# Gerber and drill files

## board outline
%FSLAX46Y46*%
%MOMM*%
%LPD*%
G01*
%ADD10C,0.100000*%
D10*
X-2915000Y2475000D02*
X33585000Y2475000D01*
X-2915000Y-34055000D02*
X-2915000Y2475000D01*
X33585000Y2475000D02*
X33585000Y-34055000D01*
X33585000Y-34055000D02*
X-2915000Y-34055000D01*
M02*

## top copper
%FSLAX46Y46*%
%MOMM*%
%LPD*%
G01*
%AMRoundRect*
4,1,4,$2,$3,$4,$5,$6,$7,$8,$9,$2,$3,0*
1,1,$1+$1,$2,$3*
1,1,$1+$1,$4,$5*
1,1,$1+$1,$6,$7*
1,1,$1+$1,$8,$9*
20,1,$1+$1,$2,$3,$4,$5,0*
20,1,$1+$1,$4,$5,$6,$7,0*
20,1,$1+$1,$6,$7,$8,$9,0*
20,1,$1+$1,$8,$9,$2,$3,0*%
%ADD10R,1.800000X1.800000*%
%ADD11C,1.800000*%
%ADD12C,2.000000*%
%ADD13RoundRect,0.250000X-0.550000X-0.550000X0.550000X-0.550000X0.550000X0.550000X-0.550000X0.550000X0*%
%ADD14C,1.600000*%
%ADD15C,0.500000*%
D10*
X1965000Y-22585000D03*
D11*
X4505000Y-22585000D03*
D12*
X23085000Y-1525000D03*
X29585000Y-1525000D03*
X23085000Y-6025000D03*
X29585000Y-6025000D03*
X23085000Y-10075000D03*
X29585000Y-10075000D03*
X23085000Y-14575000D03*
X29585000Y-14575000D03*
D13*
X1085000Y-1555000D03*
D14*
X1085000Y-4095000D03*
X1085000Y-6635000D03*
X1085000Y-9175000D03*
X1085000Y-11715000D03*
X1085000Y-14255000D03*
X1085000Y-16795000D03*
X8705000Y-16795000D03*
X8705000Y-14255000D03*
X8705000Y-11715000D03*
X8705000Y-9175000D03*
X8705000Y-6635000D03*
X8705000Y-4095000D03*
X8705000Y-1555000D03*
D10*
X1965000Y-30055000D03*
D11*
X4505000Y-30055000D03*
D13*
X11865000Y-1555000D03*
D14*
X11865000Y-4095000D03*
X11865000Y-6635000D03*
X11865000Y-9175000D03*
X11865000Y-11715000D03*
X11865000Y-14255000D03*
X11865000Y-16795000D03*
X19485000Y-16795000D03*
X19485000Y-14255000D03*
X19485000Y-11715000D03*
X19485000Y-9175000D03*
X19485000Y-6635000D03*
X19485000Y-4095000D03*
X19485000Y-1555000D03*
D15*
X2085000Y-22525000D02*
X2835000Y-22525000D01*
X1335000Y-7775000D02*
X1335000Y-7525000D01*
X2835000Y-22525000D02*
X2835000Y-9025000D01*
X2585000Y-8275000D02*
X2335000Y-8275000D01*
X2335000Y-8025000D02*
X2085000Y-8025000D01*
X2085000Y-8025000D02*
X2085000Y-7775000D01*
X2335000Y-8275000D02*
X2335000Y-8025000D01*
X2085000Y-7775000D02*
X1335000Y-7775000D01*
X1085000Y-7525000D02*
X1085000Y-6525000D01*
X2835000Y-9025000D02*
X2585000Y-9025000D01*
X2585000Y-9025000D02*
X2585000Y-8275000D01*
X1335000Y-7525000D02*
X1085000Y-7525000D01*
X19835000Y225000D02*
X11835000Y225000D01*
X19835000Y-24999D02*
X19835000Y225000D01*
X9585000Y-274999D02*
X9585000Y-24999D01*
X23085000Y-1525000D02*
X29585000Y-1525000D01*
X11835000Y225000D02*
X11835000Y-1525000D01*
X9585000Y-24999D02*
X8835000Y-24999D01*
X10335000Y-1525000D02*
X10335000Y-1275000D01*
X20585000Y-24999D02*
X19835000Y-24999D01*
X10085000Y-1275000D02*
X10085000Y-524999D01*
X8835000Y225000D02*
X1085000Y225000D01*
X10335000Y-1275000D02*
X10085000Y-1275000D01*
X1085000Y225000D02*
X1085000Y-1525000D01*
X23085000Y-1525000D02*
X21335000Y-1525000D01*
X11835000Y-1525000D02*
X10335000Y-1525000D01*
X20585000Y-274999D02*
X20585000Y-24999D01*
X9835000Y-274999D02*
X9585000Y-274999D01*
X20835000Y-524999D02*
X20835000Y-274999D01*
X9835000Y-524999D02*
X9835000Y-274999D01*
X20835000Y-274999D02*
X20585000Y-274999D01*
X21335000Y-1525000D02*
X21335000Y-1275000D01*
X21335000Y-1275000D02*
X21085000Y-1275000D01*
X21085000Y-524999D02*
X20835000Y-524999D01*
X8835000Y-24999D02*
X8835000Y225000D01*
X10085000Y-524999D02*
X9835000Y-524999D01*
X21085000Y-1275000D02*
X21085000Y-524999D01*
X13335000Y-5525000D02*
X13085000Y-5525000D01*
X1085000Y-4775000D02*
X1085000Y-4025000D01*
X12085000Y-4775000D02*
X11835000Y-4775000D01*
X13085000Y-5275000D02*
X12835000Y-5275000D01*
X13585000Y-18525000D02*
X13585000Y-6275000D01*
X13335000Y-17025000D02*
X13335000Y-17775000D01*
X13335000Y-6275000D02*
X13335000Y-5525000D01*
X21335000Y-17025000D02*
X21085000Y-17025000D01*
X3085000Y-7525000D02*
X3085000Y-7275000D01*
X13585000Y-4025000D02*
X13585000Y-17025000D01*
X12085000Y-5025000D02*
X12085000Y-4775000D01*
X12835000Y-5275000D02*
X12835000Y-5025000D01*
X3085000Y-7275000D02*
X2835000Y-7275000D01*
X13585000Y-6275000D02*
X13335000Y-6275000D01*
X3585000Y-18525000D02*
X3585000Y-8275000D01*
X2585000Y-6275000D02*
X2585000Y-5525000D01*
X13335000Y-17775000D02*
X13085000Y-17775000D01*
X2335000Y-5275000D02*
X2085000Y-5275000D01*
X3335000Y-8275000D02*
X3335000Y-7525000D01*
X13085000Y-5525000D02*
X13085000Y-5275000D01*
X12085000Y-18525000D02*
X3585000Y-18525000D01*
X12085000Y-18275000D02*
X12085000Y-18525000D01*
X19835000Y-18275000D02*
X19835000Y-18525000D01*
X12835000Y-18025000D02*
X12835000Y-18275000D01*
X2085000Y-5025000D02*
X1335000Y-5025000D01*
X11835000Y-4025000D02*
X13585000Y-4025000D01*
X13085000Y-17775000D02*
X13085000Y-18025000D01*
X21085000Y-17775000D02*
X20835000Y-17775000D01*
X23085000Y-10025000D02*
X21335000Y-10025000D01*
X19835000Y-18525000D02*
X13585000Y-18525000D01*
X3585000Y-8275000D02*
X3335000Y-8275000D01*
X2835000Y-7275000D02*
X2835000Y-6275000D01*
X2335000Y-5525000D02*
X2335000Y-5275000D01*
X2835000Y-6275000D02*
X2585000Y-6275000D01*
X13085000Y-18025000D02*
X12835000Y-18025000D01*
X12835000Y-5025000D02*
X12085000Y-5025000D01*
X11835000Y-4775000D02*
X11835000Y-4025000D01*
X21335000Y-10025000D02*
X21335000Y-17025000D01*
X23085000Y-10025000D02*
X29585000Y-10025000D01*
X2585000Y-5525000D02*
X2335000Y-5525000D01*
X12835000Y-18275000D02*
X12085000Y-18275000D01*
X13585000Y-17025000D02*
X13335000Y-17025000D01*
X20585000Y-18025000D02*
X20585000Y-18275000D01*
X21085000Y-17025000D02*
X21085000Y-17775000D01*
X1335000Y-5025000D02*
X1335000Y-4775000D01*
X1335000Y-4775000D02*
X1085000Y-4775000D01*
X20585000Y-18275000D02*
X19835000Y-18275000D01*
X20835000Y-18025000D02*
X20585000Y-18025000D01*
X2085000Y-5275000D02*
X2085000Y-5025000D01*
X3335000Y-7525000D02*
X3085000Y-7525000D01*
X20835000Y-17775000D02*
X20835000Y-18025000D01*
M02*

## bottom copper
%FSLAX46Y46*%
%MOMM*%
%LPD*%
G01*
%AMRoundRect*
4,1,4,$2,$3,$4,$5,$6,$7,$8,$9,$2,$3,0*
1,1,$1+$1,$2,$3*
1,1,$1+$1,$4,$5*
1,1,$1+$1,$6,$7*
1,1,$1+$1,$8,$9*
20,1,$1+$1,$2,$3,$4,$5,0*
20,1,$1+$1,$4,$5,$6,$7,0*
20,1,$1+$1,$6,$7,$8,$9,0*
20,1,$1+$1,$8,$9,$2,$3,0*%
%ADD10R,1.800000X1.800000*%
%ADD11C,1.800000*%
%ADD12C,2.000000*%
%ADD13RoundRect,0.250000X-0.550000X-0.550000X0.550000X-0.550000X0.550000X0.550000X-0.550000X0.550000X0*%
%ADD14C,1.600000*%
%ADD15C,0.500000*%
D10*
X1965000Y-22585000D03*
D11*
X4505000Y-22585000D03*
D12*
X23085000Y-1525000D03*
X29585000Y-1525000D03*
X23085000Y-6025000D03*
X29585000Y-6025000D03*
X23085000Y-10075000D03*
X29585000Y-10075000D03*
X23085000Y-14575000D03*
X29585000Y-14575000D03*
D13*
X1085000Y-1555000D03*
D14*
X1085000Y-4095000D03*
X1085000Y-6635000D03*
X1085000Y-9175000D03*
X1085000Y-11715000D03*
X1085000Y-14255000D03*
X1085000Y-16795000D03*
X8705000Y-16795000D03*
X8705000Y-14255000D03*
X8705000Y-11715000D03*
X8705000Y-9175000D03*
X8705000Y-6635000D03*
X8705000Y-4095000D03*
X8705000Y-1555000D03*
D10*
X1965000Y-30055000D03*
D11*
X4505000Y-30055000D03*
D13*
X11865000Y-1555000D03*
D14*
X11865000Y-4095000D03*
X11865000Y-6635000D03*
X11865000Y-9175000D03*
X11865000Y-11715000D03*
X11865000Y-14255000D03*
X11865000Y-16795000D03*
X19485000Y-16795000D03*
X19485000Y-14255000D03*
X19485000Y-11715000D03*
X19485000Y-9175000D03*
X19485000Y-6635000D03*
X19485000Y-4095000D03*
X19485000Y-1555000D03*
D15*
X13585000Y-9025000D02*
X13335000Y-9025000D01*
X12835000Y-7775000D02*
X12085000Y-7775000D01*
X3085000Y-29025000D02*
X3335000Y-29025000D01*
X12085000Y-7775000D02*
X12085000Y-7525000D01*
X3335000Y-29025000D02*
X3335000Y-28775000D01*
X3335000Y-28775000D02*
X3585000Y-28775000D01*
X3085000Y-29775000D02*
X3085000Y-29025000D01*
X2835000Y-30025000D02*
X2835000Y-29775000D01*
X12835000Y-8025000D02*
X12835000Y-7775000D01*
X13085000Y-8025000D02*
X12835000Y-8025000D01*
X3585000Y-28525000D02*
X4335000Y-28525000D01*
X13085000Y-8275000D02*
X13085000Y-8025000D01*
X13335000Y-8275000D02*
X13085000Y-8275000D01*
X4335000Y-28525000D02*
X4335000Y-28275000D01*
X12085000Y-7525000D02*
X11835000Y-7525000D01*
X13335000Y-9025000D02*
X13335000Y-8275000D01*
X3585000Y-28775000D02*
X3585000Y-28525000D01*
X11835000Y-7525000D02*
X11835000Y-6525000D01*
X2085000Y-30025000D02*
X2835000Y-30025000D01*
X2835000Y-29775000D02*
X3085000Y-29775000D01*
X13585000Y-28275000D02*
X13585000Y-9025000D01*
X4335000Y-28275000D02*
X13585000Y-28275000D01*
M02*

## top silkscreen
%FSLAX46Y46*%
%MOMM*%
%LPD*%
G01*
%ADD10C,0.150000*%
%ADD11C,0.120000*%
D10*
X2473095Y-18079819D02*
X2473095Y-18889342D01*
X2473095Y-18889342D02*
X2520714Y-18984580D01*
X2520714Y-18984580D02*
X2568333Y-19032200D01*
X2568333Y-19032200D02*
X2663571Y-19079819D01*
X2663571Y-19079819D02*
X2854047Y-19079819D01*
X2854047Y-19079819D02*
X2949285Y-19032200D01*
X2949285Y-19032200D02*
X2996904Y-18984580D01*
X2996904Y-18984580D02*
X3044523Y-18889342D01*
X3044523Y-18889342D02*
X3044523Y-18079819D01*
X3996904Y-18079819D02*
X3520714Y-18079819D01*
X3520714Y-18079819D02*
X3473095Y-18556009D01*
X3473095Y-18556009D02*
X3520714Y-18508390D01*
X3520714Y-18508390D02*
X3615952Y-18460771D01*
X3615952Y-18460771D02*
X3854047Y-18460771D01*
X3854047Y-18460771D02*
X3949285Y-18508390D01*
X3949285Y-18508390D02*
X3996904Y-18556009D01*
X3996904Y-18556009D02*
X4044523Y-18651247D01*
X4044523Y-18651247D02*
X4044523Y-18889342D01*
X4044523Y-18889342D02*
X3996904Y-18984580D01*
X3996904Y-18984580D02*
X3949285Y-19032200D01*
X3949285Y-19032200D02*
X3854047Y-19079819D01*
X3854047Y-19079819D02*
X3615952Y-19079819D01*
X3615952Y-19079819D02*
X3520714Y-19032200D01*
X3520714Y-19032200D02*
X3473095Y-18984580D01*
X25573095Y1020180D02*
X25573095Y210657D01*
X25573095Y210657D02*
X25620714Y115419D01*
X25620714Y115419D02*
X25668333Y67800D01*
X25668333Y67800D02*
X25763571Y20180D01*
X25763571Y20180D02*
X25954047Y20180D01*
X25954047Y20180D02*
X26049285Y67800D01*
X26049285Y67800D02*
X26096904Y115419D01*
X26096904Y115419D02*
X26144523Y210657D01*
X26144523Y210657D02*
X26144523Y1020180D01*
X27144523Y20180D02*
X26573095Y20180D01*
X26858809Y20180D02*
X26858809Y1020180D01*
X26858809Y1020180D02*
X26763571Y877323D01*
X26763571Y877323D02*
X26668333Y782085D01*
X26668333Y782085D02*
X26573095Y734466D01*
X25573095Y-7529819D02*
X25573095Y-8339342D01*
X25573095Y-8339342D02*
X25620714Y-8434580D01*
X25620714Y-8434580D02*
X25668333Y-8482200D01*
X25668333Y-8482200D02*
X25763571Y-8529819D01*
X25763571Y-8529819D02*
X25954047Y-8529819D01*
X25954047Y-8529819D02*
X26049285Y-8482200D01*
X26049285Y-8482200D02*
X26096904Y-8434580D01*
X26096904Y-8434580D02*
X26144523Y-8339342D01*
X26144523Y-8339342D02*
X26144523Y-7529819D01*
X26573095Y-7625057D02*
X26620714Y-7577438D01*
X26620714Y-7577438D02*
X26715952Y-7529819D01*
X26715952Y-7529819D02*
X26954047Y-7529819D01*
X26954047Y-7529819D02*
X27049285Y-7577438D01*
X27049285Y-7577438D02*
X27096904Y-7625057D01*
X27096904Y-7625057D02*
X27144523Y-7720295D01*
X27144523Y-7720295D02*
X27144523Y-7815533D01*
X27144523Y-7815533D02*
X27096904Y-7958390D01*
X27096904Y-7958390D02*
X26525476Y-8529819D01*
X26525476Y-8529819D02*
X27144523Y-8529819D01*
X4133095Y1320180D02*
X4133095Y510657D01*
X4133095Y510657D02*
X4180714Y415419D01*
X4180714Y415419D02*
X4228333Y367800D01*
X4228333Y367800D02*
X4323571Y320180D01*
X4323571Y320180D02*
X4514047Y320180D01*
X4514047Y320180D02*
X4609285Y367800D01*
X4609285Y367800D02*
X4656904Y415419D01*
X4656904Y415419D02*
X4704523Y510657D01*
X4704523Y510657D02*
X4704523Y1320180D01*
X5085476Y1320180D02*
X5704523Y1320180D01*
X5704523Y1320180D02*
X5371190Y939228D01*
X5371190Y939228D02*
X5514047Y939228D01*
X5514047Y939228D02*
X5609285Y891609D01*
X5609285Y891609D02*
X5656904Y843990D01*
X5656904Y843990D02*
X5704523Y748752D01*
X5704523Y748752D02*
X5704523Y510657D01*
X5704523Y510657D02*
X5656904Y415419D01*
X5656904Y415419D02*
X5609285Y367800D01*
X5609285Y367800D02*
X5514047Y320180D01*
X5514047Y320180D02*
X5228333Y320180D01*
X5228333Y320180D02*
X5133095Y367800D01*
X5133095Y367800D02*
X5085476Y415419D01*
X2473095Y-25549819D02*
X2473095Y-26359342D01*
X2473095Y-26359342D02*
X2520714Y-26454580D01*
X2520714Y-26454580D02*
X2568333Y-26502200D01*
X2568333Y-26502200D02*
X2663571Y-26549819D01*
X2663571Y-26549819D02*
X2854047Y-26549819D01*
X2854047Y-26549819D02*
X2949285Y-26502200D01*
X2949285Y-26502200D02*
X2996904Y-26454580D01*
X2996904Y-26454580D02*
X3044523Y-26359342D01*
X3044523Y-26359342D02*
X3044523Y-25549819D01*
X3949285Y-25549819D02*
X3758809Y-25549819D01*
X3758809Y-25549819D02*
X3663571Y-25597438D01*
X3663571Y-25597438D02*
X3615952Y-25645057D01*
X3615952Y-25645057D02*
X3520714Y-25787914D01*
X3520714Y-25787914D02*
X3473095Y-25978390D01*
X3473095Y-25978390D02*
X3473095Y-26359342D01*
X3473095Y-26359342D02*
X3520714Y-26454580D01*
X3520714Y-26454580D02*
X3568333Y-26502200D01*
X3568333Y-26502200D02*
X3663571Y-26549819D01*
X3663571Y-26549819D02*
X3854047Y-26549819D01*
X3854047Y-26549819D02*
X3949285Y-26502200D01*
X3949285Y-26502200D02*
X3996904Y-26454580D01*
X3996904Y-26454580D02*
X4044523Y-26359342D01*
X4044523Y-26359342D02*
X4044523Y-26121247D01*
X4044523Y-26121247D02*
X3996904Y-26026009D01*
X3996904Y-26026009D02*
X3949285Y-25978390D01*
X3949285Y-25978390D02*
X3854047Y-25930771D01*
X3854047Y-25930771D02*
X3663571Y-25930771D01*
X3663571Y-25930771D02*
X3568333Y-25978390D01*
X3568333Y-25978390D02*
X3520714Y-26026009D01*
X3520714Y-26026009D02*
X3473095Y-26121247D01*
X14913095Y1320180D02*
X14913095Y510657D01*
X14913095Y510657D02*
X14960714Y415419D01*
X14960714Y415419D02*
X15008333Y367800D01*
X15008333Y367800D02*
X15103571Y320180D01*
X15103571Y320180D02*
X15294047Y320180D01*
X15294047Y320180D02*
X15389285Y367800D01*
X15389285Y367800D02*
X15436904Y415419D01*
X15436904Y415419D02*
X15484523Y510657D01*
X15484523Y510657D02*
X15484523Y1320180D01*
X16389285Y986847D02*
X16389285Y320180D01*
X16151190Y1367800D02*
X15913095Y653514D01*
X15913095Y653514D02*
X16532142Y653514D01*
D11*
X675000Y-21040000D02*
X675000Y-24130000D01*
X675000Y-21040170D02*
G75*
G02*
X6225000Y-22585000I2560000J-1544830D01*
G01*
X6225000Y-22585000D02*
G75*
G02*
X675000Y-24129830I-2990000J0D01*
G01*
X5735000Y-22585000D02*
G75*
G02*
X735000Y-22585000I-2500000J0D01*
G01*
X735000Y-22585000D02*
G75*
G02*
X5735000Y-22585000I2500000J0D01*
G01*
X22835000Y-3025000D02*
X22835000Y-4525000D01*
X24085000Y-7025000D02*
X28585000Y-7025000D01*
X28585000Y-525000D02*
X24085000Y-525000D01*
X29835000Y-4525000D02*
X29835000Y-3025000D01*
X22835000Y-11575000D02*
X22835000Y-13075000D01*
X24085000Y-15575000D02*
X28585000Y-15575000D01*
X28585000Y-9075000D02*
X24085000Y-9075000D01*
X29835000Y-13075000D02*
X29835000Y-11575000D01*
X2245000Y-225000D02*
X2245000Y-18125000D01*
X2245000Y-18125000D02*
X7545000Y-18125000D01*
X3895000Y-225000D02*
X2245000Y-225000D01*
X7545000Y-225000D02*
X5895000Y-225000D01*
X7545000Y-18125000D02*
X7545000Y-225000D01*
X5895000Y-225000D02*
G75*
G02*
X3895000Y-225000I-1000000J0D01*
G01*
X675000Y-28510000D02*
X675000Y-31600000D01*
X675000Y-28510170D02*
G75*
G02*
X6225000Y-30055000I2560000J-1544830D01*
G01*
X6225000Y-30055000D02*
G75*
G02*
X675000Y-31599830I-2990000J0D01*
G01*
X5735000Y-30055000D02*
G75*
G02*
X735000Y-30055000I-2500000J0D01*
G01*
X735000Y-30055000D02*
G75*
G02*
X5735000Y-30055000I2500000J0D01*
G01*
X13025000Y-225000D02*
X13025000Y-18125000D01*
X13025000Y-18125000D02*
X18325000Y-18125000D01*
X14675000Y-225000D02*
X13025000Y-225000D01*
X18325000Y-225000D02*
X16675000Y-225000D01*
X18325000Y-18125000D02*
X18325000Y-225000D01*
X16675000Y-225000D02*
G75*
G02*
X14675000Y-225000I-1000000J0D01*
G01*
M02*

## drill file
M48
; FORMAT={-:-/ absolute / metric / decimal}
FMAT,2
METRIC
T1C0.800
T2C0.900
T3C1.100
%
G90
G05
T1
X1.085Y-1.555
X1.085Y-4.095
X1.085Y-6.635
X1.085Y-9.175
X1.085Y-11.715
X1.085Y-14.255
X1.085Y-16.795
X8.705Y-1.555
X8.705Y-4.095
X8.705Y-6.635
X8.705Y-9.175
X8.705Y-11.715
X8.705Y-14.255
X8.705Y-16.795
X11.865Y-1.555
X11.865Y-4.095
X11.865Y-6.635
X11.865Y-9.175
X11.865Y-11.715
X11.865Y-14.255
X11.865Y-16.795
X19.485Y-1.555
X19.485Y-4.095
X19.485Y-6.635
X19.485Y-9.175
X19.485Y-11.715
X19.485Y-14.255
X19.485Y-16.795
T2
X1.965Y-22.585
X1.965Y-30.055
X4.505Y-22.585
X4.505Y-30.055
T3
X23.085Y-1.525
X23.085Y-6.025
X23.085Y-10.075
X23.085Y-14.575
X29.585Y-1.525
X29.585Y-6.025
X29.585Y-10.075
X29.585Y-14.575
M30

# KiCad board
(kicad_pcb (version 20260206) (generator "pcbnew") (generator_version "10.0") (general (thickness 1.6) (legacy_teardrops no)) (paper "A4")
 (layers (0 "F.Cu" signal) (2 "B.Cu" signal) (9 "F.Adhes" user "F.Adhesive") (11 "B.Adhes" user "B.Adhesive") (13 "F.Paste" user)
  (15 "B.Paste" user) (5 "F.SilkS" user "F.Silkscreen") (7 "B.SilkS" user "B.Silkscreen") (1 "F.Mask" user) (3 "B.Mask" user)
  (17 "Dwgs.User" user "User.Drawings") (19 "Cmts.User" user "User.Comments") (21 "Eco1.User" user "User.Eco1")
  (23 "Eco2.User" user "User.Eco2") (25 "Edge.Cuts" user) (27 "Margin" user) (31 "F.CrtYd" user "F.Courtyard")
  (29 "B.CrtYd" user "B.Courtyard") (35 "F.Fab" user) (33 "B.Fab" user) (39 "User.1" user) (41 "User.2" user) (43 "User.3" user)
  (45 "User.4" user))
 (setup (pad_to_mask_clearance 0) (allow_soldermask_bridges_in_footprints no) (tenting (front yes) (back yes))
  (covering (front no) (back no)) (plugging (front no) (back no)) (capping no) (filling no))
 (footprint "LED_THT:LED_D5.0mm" (layer "F.Cu") (at 1.965 22.585)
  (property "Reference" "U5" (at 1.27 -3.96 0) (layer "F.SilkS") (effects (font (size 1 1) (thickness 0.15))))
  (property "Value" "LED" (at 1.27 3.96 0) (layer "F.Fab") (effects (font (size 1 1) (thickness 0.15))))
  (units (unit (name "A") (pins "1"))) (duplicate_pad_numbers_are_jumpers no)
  (fp_line (start -1.29 -1.545) (end -1.29 1.545) (stroke (width 0.12) (type solid)) (layer "F.SilkS"))
  (fp_arc (start -1.29 -1.54483) (mid 2.071779 -2.880495) (end 4.26 0) (stroke (width 0.12) (type solid)) (layer "F.SilkS"))
  (fp_arc (start 4.26 0) (mid 2.071779 2.880495) (end -1.29 1.54483) (stroke (width 0.12) (type solid)) (layer "F.SilkS"))
  (fp_circle (center 1.27 0) (end 3.77 0) (stroke (width 0.12) (type solid)) (fill no) (layer "F.SilkS"))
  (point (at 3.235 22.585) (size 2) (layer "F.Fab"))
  (pad "1" thru_hole rect (at 0 0) (size 1.8 1.8) (drill 0.9) (layers "*.Cu" "*.Mask") (remove_unused_layers no) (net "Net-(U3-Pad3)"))
  (pad "2" thru_hole circle (at 2.54 0) (size 1.8 1.8) (drill 0.9) (layers "*.Cu" "*.Mask") (remove_unused_layers no)))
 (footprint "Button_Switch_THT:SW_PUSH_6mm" (layer "F.Cu") (at 23.085 1.525)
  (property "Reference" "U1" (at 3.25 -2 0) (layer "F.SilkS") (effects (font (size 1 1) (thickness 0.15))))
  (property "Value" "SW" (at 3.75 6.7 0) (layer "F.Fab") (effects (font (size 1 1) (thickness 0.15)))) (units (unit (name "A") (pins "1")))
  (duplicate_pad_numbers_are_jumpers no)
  (fp_line (start -0.25 1.5) (end -0.25 3) (stroke (width 0.12) (type solid)) (layer "F.SilkS"))
  (fp_line (start 1 5.5) (end 5.5 5.5) (stroke (width 0.12) (type solid)) (layer "F.SilkS"))
  (fp_line (start 5.5 -1) (end 1 -1) (stroke (width 0.12) (type solid)) (layer "F.SilkS"))
  (fp_line (start 6.75 3) (end 6.75 1.5) (stroke (width 0.12) (type solid)) (layer "F.SilkS"))
  (pad "1" thru_hole circle (at 0 0 90) (size 2 2) (drill 1.1) (layers "*.Cu" "*.Mask") (remove_unused_layers no) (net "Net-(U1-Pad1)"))
  (pad "1" thru_hole circle (at 6.5 0 90) (size 2 2) (drill 1.1) (layers "*.Cu" "*.Mask") (remove_unused_layers no) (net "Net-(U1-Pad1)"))
  (pad "2" thru_hole circle (at 0 4.5 90) (size 2 2) (drill 1.1) (layers "*.Cu" "*.Mask") (remove_unused_layers no))
  (pad "2" thru_hole circle (at 6.5 4.5 90) (size 2 2) (drill 1.1) (layers "*.Cu" "*.Mask") (remove_unused_layers no)))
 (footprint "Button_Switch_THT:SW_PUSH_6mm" (layer "F.Cu") (at 23.085 10.075)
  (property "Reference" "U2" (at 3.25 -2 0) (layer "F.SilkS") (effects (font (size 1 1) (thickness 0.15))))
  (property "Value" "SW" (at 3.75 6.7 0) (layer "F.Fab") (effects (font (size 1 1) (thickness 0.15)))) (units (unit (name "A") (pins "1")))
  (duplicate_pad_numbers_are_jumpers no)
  (fp_line (start -0.25 1.5) (end -0.25 3) (stroke (width 0.12) (type solid)) (layer "F.SilkS"))
  (fp_line (start 1 5.5) (end 5.5 5.5) (stroke (width 0.12) (type solid)) (layer "F.SilkS"))
  (fp_line (start 5.5 -1) (end 1 -1) (stroke (width 0.12) (type solid)) (layer "F.SilkS"))
  (fp_line (start 6.75 3) (end 6.75 1.5) (stroke (width 0.12) (type solid)) (layer "F.SilkS"))
  (pad "1" thru_hole circle (at 0 0 90) (size 2 2) (drill 1.1) (layers "*.Cu" "*.Mask") (remove_unused_layers no) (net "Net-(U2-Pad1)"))
  (pad "1" thru_hole circle (at 6.5 0 90) (size 2 2) (drill 1.1) (layers "*.Cu" "*.Mask") (remove_unused_layers no) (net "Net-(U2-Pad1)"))
  (pad "2" thru_hole circle (at 0 4.5 90) (size 2 2) (drill 1.1) (layers "*.Cu" "*.Mask") (remove_unused_layers no))
  (pad "2" thru_hole circle (at 6.5 4.5 90) (size 2 2) (drill 1.1) (layers "*.Cu" "*.Mask") (remove_unused_layers no)))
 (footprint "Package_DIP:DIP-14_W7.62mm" (layer "F.Cu") (at 1.085 1.555)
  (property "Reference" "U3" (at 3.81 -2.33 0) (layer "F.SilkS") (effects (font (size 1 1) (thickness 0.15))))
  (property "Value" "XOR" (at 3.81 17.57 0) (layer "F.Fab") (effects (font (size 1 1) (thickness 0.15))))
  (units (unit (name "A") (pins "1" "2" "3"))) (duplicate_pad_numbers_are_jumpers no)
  (fp_line (start 1.16 -1.33) (end 1.16 16.57) (stroke (width 0.12) (type solid)) (layer "F.SilkS"))
  (fp_line (start 1.16 16.57) (end 6.46 16.57) (stroke (width 0.12) (type solid)) (layer "F.SilkS"))
  (fp_line (start 2.81 -1.33) (end 1.16 -1.33) (stroke (width 0.12) (type solid)) (layer "F.SilkS"))
  (fp_line (start 6.46 -1.33) (end 4.81 -1.33) (stroke (width 0.12) (type solid)) (layer "F.SilkS"))
  (fp_line (start 6.46 16.57) (end 6.46 -1.33) (stroke (width 0.12) (type solid)) (layer "F.SilkS"))
  (fp_arc (start 4.81 -1.33) (mid 3.81 -0.33) (end 2.81 -1.33) (stroke (width 0.12) (type solid)) (layer "F.SilkS"))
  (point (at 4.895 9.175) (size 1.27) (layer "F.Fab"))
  (pad "1" thru_hole roundrect (at 0 0) (size 1.6 1.6) (drill 0.8) (layers "*.Cu" "*.Mask") (remove_unused_layers no)
   (roundrect_rratio 0.15625) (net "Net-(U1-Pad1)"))
  (pad "2" thru_hole circle (at 0 2.54) (size 1.6 1.6) (drill 0.8) (layers "*.Cu" "*.Mask") (remove_unused_layers no) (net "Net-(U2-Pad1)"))
  (pad "3" thru_hole circle (at 0 5.08) (size 1.6 1.6) (drill 0.8) (layers "*.Cu" "*.Mask") (remove_unused_layers no) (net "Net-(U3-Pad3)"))
  (pad "4" thru_hole circle (at 0 7.62) (size 1.6 1.6) (drill 0.8) (layers "*.Cu" "*.Mask") (remove_unused_layers no))
  (pad "5" thru_hole circle (at 0 10.16) (size 1.6 1.6) (drill 0.8) (layers "*.Cu" "*.Mask") (remove_unused_layers no))
  (pad "6" thru_hole circle (at 0 12.7) (size 1.6 1.6) (drill 0.8) (layers "*.Cu" "*.Mask") (remove_unused_layers no))
  (pad "7" thru_hole circle (at 0 15.24) (size 1.6 1.6) (drill 0.8) (layers "*.Cu" "*.Mask") (remove_unused_layers no))
  (pad "8" thru_hole circle (at 7.62 15.24) (size 1.6 1.6) (drill 0.8) (layers "*.Cu" "*.Mask") (remove_unused_layers no))
  (pad "9" thru_hole circle (at 7.62 12.7) (size 1.6 1.6) (drill 0.8) (layers "*.Cu" "*.Mask") (remove_unused_layers no))
  (pad "10" thru_hole circle (at 7.62 10.16) (size 1.6 1.6) (drill 0.8) (layers "*.Cu" "*.Mask") (remove_unused_layers no))
  (pad "11" thru_hole circle (at 7.62 7.62) (size 1.6 1.6) (drill 0.8) (layers "*.Cu" "*.Mask") (remove_unused_layers no))
  (pad "12" thru_hole circle (at 7.62 5.08) (size 1.6 1.6) (drill 0.8) (layers "*.Cu" "*.Mask") (remove_unused_layers no))
  (pad "13" thru_hole circle (at 7.62 2.54) (size 1.6 1.6) (drill 0.8) (layers "*.Cu" "*.Mask") (remove_unused_layers no))
  (pad "14" thru_hole circle (at 7.62 0) (size 1.6 1.6) (drill 0.8) (layers "*.Cu" "*.Mask") (remove_unused_layers no)))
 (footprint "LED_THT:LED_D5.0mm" (layer "F.Cu") (at 1.965 30.055)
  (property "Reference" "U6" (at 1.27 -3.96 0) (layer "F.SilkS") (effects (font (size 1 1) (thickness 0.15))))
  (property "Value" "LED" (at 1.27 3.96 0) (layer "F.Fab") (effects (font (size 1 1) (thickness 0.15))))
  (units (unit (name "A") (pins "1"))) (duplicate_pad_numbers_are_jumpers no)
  (fp_line (start -1.29 -1.545) (end -1.29 1.545) (stroke (width 0.12) (type solid)) (layer "F.SilkS"))
  (fp_arc (start -1.29 -1.54483) (mid 2.071779 -2.880495) (end 4.26 0) (stroke (width 0.12) (type solid)) (layer "F.SilkS"))
  (fp_arc (start 4.26 0) (mid 2.071779 2.880495) (end -1.29 1.54483) (stroke (width 0.12) (type solid)) (layer "F.SilkS"))
  (fp_circle (center 1.27 0) (end 3.77 0) (stroke (width 0.12) (type solid)) (fill no) (layer "F.SilkS"))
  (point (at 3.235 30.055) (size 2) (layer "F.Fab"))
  (pad "1" thru_hole rect (at 0 0) (size 1.8 1.8) (drill 0.9) (layers "*.Cu" "*.Mask") (remove_unused_layers no) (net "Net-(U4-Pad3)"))
  (pad "2" thru_hole circle (at 2.54 0) (size 1.8 1.8) (drill 0.9) (layers "*.Cu" "*.Mask") (remove_unused_layers no)))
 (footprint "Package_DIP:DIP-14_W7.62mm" (layer "F.Cu") (at 11.865 1.555)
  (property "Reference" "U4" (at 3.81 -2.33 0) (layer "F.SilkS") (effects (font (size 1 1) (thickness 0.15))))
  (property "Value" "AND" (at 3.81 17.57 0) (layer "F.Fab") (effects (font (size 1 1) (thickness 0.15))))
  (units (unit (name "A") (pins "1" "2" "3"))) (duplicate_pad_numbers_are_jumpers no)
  (fp_line (start 1.16 -1.33) (end 1.16 16.57) (stroke (width 0.12) (type solid)) (layer "F.SilkS"))
  (fp_line (start 1.16 16.57) (end 6.46 16.57) (stroke (width 0.12) (type solid)) (layer "F.SilkS"))
  (fp_line (start 2.81 -1.33) (end 1.16 -1.33) (stroke (width 0.12) (type solid)) (layer "F.SilkS"))
  (fp_line (start 6.46 -1.33) (end 4.81 -1.33) (stroke (width 0.12) (type solid)) (layer "F.SilkS"))
  (fp_line (start 6.46 16.57) (end 6.46 -1.33) (stroke (width 0.12) (type solid)) (layer "F.SilkS"))
  (fp_arc (start 4.81 -1.33) (mid 3.81 -0.33) (end 2.81 -1.33) (stroke (width 0.12) (type solid)) (layer "F.SilkS"))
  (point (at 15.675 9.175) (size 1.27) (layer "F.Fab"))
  (pad "1" thru_hole roundrect (at 0 0) (size 1.6 1.6) (drill 0.8) (layers "*.Cu" "*.Mask") (remove_unused_layers no)
   (roundrect_rratio 0.15625) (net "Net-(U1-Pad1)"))
  (pad "2" thru_hole circle (at 0 2.54) (size 1.6 1.6) (drill 0.8) (layers "*.Cu" "*.Mask") (remove_unused_layers no) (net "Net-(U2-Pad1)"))
  (pad "3" thru_hole circle (at 0 5.08) (size 1.6 1.6) (drill 0.8) (layers "*.Cu" "*.Mask") (remove_unused_layers no) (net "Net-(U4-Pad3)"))
  (pad "4" thru_hole circle (at 0 7.62) (size 1.6 1.6) (drill 0.8) (layers "*.Cu" "*.Mask") (remove_unused_layers no))
  (pad "5" thru_hole circle (at 0 10.16) (size 1.6 1.6) (drill 0.8) (layers "*.Cu" "*.Mask") (remove_unused_layers no))
  (pad "6" thru_hole circle (at 0 12.7) (size 1.6 1.6) (drill 0.8) (layers "*.Cu" "*.Mask") (remove_unused_layers no))
  (pad "7" thru_hole circle (at 0 15.24) (size 1.6 1.6) (drill 0.8) (layers "*.Cu" "*.Mask") (remove_unused_layers no))
  (pad "8" thru_hole circle (at 7.62 15.24) (size 1.6 1.6) (drill 0.8) (layers "*.Cu" "*.Mask") (remove_unused_layers no))
  (pad "9" thru_hole circle (at 7.62 12.7) (size 1.6 1.6) (drill 0.8) (layers "*.Cu" "*.Mask") (remove_unused_layers no))
  (pad "10" thru_hole circle (at 7.62 10.16) (size 1.6 1.6) (drill 0.8) (layers "*.Cu" "*.Mask") (remove_unused_layers no))
  (pad "11" thru_hole circle (at 7.62 7.62) (size 1.6 1.6) (drill 0.8) (layers "*.Cu" "*.Mask") (remove_unused_layers no))
  (pad "12" thru_hole circle (at 7.62 5.08) (size 1.6 1.6) (drill 0.8) (layers "*.Cu" "*.Mask") (remove_unused_layers no))
  (pad "13" thru_hole circle (at 7.62 2.54) (size 1.6 1.6) (drill 0.8) (layers "*.Cu" "*.Mask") (remove_unused_layers no))
  (pad "14" thru_hole circle (at 7.62 0) (size 1.6 1.6) (drill 0.8) (layers "*.Cu" "*.Mask") (remove_unused_layers no)))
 (gr_line (start -2.915 -2.475) (end 33.585 -2.475) (stroke (width 0.1) (type default)) (layer "Edge.Cuts"))
 (gr_line (start -2.915 34.055) (end -2.915 -2.475) (stroke (width 0.1) (type default)) (layer "Edge.Cuts"))
 (gr_line (start 33.585 -2.475) (end 33.585 34.055) (stroke (width 0.1) (type default)) (layer "Edge.Cuts"))
 (gr_line (start 33.585 34.055) (end -2.915 34.055) (stroke (width 0.1) (type default)) (layer "Edge.Cuts"))
 (segment (start 2.085 22.525) (end 2.835 22.525) (width 0.5) (layer "F.Cu") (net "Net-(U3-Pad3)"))
 (segment (start 1.335 7.775) (end 1.335 7.525) (width 0.5) (layer "F.Cu") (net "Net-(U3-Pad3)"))
 (segment (start 2.835 22.525) (end 2.835 9.025) (width 0.5) (layer "F.Cu") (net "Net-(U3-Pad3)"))
 (segment (start 2.585 8.275) (end 2.335 8.275) (width 0.5) (layer "F.Cu") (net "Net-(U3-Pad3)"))
 (segment (start 2.335 8.025) (end 2.085 8.025) (width 0.5) (layer "F.Cu") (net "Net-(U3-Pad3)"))
 (segment (start 2.085 8.025) (end 2.085 7.775) (width 0.5) (layer "F.Cu") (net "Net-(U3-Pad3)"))
 (segment (start 2.335 8.275) (end 2.335 8.025) (width 0.5) (layer "F.Cu") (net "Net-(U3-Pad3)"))
 (segment (start 2.085 7.775) (end 1.335 7.775) (width 0.5) (layer "F.Cu") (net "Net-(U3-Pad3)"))
 (segment (start 1.085 7.525) (end 1.085 6.525) (width 0.5) (layer "F.Cu") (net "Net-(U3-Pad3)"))
 (segment (start 2.835 9.025) (end 2.585 9.025) (width 0.5) (layer "F.Cu") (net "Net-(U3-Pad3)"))
 (segment (start 2.585 9.025) (end 2.585 8.275) (width 0.5) (layer "F.Cu") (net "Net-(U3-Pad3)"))
 (segment (start 1.335 7.525) (end 1.085 7.525) (width 0.5) (layer "F.Cu") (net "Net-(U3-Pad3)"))
 (segment (start 19.835 -0.225) (end 11.835 -0.225) (width 0.5) (layer "F.Cu") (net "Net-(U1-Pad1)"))
 (segment (start 19.835 0.024999) (end 19.835 -0.225) (width 0.5) (layer "F.Cu") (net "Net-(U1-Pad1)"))
 (segment (start 9.585 0.274999) (end 9.585 0.024999) (width 0.5) (layer "F.Cu") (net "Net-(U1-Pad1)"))
 (segment (start 23.085 1.525) (end 29.585 1.525) (width 0.5) (layer "F.Cu") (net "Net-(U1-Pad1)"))
 (segment (start 11.835 -0.225) (end 11.835 1.525) (width 0.5) (layer "F.Cu") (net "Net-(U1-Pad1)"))
 (segment (start 9.585 0.024999) (end 8.835 0.024999) (width 0.5) (layer "F.Cu") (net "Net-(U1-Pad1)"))
 (segment (start 10.335 1.525) (end 10.335 1.275) (width 0.5) (layer "F.Cu") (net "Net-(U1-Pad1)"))
 (segment (start 20.585 0.024999) (end 19.835 0.024999) (width 0.5) (layer "F.Cu") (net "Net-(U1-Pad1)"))
 (segment (start 10.085 1.275) (end 10.085 0.524999) (width 0.5) (layer "F.Cu") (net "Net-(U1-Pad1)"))
 (segment (start 8.835 -0.225) (end 1.085 -0.225) (width 0.5) (layer "F.Cu") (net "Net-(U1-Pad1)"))
 (segment (start 10.335 1.275) (end 10.085 1.275) (width 0.5) (layer "F.Cu") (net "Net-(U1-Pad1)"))
 (segment (start 1.085 -0.225) (end 1.085 1.525) (width 0.5) (layer "F.Cu") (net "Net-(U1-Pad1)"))
 (segment (start 23.085 1.525) (end 21.335 1.525) (width 0.5) (layer "F.Cu") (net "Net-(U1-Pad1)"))
 (segment (start 11.835 1.525) (end 10.335 1.525) (width 0.5) (layer "F.Cu") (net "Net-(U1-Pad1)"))
 (segment (start 20.585 0.274999) (end 20.585 0.024999) (width 0.5) (layer "F.Cu") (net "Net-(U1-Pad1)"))
 (segment (start 9.835 0.274999) (end 9.585 0.274999) (width 0.5) (layer "F.Cu") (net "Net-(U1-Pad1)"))
 (segment (start 20.835 0.524999) (end 20.835 0.274999) (width 0.5) (layer "F.Cu") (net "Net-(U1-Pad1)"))
 (segment (start 9.835 0.524999) (end 9.835 0.274999) (width 0.5) (layer "F.Cu") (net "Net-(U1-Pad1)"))
 (segment (start 20.835 0.274999) (end 20.585 0.274999) (width 0.5) (layer "F.Cu") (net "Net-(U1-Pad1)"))
 (segment (start 21.335 1.525) (end 21.335 1.275) (width 0.5) (layer "F.Cu") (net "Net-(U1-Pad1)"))
 (segment (start 21.335 1.275) (end 21.085 1.275) (width 0.5) (layer "F.Cu") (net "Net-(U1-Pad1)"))
 (segment (start 21.085 0.524999) (end 20.835 0.524999) (width 0.5) (layer "F.Cu") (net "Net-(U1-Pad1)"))
 (segment (start 8.835 0.024999) (end 8.835 -0.225) (width 0.5) (layer "F.Cu") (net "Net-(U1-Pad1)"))
 (segment (start 10.085 0.524999) (end 9.835 0.524999) (width 0.5) (layer "F.Cu") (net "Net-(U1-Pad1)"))
 (segment (start 21.085 1.275) (end 21.085 0.524999) (width 0.5) (layer "F.Cu") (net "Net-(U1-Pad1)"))
 (segment (start 13.335 5.525) (end 13.085 5.525) (width 0.5) (layer "F.Cu") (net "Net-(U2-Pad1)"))
 (segment (start 1.085 4.775) (end 1.085 4.025) (width 0.5) (layer "F.Cu") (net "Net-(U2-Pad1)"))
 (segment (start 12.085 4.775) (end 11.835 4.775) (width 0.5) (layer "F.Cu") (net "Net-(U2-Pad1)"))
 (segment (start 13.085 5.275) (end 12.835 5.275) (width 0.5) (layer "F.Cu") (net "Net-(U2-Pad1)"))
 (segment (start 13.585 18.525) (end 13.585 6.275) (width 0.5) (layer "F.Cu") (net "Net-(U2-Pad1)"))
 (segment (start 13.335 17.025) (end 13.335 17.775) (width 0.5) (layer "F.Cu") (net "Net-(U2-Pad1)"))
 (segment (start 13.335 6.275) (end 13.335 5.525) (width 0.5) (layer "F.Cu") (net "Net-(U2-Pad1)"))
 (segment (start 21.335 17.025) (end 21.085 17.025) (width 0.5) (layer "F.Cu") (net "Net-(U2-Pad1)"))
 (segment (start 3.085 7.525) (end 3.085 7.275) (width 0.5) (layer "F.Cu") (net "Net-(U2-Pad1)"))
 (segment (start 13.585 4.025) (end 13.585 17.025) (width 0.5) (layer "F.Cu") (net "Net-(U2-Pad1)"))
 (segment (start 12.085 5.025) (end 12.085 4.775) (width 0.5) (layer "F.Cu") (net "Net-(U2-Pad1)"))
 (segment (start 12.835 5.275) (end 12.835 5.025) (width 0.5) (layer "F.Cu") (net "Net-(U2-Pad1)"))
 (segment (start 3.085 7.275) (end 2.835 7.275) (width 0.5) (layer "F.Cu") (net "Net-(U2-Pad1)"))
 (segment (start 13.585 6.275) (end 13.335 6.275) (width 0.5) (layer "F.Cu") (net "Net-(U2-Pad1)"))
 (segment (start 3.585 18.525) (end 3.585 8.275) (width 0.5) (layer "F.Cu") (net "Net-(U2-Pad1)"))
 (segment (start 2.585 6.275) (end 2.585 5.525) (width 0.5) (layer "F.Cu") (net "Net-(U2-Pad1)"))
 (segment (start 13.335 17.775) (end 13.085 17.775) (width 0.5) (layer "F.Cu") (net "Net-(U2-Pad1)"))
 (segment (start 2.335 5.275) (end 2.085 5.275) (width 0.5) (layer "F.Cu") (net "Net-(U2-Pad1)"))
 (segment (start 3.335 8.275) (end 3.335 7.525) (width 0.5) (layer "F.Cu") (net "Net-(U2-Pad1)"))
 (segment (start 13.085 5.525) (end 13.085 5.275) (width 0.5) (layer "F.Cu") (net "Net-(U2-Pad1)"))
 (segment (start 12.085 18.525) (end 3.585 18.525) (width 0.5) (layer "F.Cu") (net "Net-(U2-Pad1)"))
 (segment (start 12.085 18.275) (end 12.085 18.525) (width 0.5) (layer "F.Cu") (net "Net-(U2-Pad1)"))
 (segment (start 19.835 18.275) (end 19.835 18.525) (width 0.5) (layer "F.Cu") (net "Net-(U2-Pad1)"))
 (segment (start 12.835 18.025) (end 12.835 18.275) (width 0.5) (layer "F.Cu") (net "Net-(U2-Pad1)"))
 (segment (start 2.085 5.025) (end 1.335 5.025) (width 0.5) (layer "F.Cu") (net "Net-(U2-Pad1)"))
 (segment (start 11.835 4.025) (end 13.585 4.025) (width 0.5) (layer "F.Cu") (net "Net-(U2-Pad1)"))
 (segment (start 13.085 17.775) (end 13.085 18.025) (width 0.5) (layer "F.Cu") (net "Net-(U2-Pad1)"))
 (segment (start 21.085 17.775) (end 20.835 17.775) (width 0.5) (layer "F.Cu") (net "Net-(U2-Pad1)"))
 (segment (start 23.085 10.025) (end 21.335 10.025) (width 0.5) (layer "F.Cu") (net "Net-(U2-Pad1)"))
 (segment (start 19.835 18.525) (end 13.585 18.525) (width 0.5) (layer "F.Cu") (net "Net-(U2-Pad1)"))
 (segment (start 3.585 8.275) (end 3.335 8.275) (width 0.5) (layer "F.Cu") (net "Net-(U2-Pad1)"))
 (segment (start 2.835 7.275) (end 2.835 6.275) (width 0.5) (layer "F.Cu") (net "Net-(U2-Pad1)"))
 (segment (start 2.335 5.525) (end 2.335 5.275) (width 0.5) (layer "F.Cu") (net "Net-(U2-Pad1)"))
 (segment (start 2.835 6.275) (end 2.585 6.275) (width 0.5) (layer "F.Cu") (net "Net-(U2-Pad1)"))
 (segment (start 13.085 18.025) (end 12.835 18.025) (width 0.5) (layer "F.Cu") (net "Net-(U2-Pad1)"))
 (segment (start 12.835 5.025) (end 12.085 5.025) (width 0.5) (layer "F.Cu") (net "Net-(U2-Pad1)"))
 (segment (start 11.835 4.775) (end 11.835 4.025) (width 0.5) (layer "F.Cu") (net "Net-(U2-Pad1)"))
 (segment (start 21.335 10.025) (end 21.335 17.025) (width 0.5) (layer "F.Cu") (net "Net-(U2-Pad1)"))
 (segment (start 23.085 10.025) (end 29.585 10.025) (width 0.5) (layer "F.Cu") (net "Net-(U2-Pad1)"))
 (segment (start 2.585 5.525) (end 2.335 5.525) (width 0.5) (layer "F.Cu") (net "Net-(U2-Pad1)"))
 (segment (start 12.835 18.275) (end 12.085 18.275) (width 0.5) (layer "F.Cu") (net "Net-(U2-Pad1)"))
 (segment (start 13.585 17.025) (end 13.335 17.025) (width 0.5) (layer "F.Cu") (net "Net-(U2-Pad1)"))
 (segment (start 20.585 18.025) (end 20.585 18.275) (width 0.5) (layer "F.Cu") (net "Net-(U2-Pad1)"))
 (segment (start 21.085 17.025) (end 21.085 17.775) (width 0.5) (layer "F.Cu") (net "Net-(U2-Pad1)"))
 (segment (start 1.335 5.025) (end 1.335 4.775) (width 0.5) (layer "F.Cu") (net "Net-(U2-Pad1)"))
 (segment (start 1.335 4.775) (end 1.085 4.775) (width 0.5) (layer "F.Cu") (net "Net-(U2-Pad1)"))
 (segment (start 20.585 18.275) (end 19.835 18.275) (width 0.5) (layer "F.Cu") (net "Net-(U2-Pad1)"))
 (segment (start 20.835 18.025) (end 20.585 18.025) (width 0.5) (layer "F.Cu") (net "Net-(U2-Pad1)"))
 (segment (start 2.085 5.275) (end 2.085 5.025) (width 0.5) (layer "F.Cu") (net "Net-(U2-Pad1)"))
 (segment (start 3.335 7.525) (end 3.085 7.525) (width 0.5) (layer "F.Cu") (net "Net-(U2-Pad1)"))
 (segment (start 20.835 17.775) (end 20.835 18.025) (width 0.5) (layer "F.Cu") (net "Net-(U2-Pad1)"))
 (segment (start 13.585 9.025) (end 13.335 9.025) (width 0.5) (layer "B.Cu") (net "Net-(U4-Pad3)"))
 (segment (start 12.835 7.775) (end 12.085 7.775) (width 0.5) (layer "B.Cu") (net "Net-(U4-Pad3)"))
 (segment (start 3.085 29.025) (end 3.335 29.025) (width 0.5) (layer "B.Cu") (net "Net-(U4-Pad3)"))
 (segment (start 12.085 7.775) (end 12.085 7.525) (width 0.5) (layer "B.Cu") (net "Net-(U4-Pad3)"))
 (segment (start 3.335 29.025) (end 3.335 28.775) (width 0.5) (layer "B.Cu") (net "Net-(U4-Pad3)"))
 (segment (start 3.335 28.775) (end 3.585 28.775) (width 0.5) (layer "B.Cu") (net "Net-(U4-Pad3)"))
 (segment (start 3.085 29.775) (end 3.085 29.025) (width 0.5) (layer "B.Cu") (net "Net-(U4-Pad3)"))
 (segment (start 2.835 30.025) (end 2.835 29.775) (width 0.5) (layer "B.Cu") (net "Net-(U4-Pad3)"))
 (segment (start 12.835 8.025) (end 12.835 7.775) (width 0.5) (layer "B.Cu") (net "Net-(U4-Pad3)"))
 (segment (start 13.085 8.025) (end 12.835 8.025) (width 0.5) (layer "B.Cu") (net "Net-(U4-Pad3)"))
 (segment (start 3.585 28.525) (end 4.335 28.525) (width 0.5) (layer "B.Cu") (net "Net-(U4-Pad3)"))
 (segment (start 13.085 8.275) (end 13.085 8.025) (width 0.5) (layer "B.Cu") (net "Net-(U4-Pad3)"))
 (segment (start 13.335 8.275) (end 13.085 8.275) (width 0.5) (layer "B.Cu") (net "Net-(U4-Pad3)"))
 (segment (start 4.335 28.525) (end 4.335 28.275) (width 0.5) (layer "B.Cu") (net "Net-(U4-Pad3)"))
 (segment (start 12.085 7.525) (end 11.835 7.525) (width 0.5) (layer "B.Cu") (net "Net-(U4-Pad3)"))
 (segment (start 13.335 9.025) (end 13.335 8.275) (width 0.5) (layer "B.Cu") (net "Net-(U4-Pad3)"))
 (segment (start 3.585 28.775) (end 3.585 28.525) (width 0.5) (layer "B.Cu") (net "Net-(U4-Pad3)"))
 (segment (start 11.835 7.525) (end 11.835 6.525) (width 0.5) (layer "B.Cu") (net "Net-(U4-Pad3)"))
 (segment (start 2.085 30.025) (end 2.835 30.025) (width 0.5) (layer "B.Cu") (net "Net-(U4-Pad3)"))
 (segment (start 2.835 29.775) (end 3.085 29.775) (width 0.5) (layer "B.Cu") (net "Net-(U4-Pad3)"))
 (segment (start 13.585 28.275) (end 13.585 9.025) (width 0.5) (layer "B.Cu") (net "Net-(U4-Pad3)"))
 (segment (start 4.335 28.275) (end 13.585 28.275) (width 0.5) (layer "B.Cu") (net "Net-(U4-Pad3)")))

